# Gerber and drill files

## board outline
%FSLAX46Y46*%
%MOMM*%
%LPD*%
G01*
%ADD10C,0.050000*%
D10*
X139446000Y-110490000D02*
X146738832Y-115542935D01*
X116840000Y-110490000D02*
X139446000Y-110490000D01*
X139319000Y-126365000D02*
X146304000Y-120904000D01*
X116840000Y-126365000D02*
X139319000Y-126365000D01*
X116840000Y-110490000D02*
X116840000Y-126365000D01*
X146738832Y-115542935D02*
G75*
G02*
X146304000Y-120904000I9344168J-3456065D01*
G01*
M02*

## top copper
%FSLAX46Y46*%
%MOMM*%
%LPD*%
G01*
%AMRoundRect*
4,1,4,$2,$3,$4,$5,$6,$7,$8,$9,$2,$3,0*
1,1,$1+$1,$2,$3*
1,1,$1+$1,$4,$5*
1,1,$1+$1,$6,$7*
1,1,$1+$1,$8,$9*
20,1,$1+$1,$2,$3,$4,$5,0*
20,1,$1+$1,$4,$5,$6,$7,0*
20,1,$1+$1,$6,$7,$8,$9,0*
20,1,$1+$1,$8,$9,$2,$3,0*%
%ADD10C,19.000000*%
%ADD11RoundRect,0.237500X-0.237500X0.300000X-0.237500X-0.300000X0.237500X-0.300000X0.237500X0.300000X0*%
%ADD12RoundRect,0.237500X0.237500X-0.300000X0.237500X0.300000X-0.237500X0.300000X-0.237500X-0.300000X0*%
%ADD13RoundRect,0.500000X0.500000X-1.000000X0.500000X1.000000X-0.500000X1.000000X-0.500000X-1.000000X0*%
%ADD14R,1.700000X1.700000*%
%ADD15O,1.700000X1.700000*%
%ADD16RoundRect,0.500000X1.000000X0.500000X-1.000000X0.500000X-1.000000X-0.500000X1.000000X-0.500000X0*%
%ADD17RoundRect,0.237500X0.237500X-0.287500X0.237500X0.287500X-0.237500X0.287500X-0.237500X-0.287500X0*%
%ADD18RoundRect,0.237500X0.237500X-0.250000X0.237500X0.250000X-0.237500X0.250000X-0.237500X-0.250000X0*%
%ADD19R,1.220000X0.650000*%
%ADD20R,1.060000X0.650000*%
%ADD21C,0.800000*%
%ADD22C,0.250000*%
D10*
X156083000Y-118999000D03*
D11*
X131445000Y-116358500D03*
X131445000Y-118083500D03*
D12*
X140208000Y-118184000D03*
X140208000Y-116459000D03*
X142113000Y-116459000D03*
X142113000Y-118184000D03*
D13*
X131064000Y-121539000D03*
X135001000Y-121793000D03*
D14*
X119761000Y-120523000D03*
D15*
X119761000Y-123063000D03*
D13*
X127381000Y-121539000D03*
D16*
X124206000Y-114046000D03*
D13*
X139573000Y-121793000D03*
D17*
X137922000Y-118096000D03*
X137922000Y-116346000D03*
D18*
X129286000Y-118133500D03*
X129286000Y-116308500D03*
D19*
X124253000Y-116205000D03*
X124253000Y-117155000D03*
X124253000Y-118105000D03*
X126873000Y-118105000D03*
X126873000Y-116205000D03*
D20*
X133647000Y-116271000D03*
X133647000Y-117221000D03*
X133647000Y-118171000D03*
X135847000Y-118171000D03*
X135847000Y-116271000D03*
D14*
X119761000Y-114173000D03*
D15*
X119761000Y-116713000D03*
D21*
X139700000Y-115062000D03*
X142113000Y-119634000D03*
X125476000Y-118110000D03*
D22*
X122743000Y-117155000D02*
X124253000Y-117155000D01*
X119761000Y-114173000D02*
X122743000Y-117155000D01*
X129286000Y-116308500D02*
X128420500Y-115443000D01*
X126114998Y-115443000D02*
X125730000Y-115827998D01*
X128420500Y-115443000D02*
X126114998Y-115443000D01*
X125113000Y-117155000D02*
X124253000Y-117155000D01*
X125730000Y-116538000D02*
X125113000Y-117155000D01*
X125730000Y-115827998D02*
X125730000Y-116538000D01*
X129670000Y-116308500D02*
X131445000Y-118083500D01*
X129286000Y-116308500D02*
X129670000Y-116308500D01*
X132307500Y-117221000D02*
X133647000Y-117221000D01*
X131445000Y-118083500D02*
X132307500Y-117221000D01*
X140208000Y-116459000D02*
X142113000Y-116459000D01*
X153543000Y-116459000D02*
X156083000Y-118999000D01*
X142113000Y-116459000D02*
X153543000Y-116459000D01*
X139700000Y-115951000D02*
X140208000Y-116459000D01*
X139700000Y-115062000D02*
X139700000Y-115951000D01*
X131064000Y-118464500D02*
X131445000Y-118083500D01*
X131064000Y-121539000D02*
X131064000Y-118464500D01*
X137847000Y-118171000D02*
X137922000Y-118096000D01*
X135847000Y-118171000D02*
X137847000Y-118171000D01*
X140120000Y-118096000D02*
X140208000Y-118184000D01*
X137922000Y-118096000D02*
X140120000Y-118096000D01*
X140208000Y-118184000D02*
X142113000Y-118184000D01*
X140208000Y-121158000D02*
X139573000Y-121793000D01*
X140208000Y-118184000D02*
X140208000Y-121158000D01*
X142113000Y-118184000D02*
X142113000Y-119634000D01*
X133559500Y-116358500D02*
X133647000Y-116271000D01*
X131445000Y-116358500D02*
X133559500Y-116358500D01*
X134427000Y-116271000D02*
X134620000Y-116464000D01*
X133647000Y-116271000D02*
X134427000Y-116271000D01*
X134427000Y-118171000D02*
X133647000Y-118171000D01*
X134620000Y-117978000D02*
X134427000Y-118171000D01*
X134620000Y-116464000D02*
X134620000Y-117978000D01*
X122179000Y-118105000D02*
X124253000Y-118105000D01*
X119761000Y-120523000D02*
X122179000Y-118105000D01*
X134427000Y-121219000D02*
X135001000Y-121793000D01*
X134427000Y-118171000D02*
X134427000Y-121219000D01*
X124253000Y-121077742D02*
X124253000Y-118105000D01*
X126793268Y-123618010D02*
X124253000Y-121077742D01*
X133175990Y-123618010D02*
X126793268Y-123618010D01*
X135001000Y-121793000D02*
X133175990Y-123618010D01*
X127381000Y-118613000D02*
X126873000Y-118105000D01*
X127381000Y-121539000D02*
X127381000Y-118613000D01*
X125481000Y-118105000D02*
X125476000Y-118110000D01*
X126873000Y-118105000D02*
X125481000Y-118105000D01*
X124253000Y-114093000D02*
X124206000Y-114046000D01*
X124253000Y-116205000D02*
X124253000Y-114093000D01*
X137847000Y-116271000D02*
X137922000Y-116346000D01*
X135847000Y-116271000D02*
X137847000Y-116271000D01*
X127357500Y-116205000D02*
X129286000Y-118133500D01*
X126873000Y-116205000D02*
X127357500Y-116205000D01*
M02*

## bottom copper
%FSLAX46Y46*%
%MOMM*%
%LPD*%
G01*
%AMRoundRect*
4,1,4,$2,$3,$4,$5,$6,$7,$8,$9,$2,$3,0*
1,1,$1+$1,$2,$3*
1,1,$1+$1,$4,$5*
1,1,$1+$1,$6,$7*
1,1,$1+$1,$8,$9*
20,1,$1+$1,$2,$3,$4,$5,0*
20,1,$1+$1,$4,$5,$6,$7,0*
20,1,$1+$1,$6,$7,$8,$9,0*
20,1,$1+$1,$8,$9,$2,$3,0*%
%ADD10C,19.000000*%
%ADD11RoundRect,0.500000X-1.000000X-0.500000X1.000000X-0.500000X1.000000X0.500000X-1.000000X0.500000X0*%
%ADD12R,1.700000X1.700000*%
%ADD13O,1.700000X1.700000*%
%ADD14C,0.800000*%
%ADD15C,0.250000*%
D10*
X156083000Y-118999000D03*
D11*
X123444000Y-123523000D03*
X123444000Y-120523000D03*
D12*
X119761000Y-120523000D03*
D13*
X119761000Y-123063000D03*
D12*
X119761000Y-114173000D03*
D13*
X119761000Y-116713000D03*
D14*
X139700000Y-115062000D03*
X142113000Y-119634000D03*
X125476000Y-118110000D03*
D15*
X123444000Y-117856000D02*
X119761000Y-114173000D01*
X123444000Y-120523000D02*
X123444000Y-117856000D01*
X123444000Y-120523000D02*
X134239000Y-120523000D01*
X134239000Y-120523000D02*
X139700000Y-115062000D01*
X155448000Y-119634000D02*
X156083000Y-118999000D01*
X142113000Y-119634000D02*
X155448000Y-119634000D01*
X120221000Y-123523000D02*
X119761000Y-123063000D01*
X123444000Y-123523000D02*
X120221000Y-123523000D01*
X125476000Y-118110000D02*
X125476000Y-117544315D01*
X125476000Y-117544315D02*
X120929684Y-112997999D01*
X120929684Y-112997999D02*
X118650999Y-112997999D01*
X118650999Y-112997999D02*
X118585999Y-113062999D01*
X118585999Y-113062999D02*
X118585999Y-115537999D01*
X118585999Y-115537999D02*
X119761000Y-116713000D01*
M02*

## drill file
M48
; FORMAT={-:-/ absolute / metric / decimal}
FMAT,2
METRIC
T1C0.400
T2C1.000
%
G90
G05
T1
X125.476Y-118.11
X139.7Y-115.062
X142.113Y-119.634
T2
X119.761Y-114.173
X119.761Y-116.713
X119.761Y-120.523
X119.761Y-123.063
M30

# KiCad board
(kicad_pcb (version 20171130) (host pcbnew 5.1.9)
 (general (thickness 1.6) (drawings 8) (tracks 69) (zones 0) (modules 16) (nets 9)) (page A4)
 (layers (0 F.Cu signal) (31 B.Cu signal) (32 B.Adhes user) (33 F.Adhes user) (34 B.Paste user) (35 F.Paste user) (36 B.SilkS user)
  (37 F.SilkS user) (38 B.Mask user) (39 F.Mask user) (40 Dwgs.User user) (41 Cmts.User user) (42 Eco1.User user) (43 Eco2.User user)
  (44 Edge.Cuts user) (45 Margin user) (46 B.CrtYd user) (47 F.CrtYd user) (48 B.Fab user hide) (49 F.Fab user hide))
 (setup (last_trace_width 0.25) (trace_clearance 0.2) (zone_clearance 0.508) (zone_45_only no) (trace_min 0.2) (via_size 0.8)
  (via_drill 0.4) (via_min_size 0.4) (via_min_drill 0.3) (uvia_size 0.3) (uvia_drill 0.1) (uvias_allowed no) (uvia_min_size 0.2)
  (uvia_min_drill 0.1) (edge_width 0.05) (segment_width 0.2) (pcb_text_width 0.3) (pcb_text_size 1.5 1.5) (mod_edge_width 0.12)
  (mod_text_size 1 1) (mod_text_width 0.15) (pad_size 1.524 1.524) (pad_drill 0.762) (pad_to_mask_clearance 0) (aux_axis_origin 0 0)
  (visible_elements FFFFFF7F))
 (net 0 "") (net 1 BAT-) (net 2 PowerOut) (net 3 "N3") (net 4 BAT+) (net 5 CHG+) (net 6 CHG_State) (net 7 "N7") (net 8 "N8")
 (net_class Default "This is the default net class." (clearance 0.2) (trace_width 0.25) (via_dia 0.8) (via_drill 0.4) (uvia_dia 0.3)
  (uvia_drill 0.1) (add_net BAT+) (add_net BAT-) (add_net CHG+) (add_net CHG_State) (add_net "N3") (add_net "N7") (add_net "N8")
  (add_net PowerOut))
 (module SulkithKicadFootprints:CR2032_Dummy (layer F.Cu) (at 156.083 118.999)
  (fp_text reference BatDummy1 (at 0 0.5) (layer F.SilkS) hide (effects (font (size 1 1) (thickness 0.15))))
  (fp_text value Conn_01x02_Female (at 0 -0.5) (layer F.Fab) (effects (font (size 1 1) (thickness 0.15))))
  (pad 1 smd circle (at 0 0) (size 19 19) (layers F.Cu F.Paste F.Mask) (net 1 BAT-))
  (pad 2 smd circle (at 0 0) (size 19 19) (layers B.Cu B.Paste B.Mask) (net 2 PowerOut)))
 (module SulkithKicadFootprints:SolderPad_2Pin (layer B.Cu) (at 123.444 123.523)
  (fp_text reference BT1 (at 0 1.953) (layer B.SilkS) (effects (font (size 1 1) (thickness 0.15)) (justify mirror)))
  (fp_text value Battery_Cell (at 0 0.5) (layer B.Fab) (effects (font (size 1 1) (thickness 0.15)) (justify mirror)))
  (pad 1 smd roundrect (at 0 0) (size 3 2) (layers B.Cu B.Paste B.Mask) (roundrect_rratio 0.25) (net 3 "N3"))
  (pad 2 smd roundrect (at 0 -3) (size 3 2) (layers B.Cu B.Paste B.Mask) (roundrect_rratio 0.25) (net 1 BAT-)))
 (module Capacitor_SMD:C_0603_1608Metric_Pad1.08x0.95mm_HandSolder (layer F.Cu) (at 131.445 117.221 270)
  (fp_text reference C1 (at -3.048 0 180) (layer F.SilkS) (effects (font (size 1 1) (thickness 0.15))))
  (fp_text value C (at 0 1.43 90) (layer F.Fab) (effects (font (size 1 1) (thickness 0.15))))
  (pad 1 smd roundrect (at -0.8625 0 270) (size 1.075 0.95) (layers F.Cu F.Paste F.Mask) (roundrect_rratio 0.25) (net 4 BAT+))
  (pad 2 smd roundrect (at 0.8625 0 270) (size 1.075 0.95) (layers F.Cu F.Paste F.Mask) (roundrect_rratio 0.25) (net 1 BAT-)))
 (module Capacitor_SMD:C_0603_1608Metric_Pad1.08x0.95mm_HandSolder (layer F.Cu) (at 140.208 117.3215 90)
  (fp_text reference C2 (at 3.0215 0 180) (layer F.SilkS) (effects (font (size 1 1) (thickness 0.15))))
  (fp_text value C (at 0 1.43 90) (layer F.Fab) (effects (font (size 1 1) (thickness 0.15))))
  (pad 1 smd roundrect (at -0.8625 0 90) (size 1.075 0.95) (layers F.Cu F.Paste F.Mask) (roundrect_rratio 0.25) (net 2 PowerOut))
  (pad 2 smd roundrect (at 0.8625 0 90) (size 1.075 0.95) (layers F.Cu F.Paste F.Mask) (roundrect_rratio 0.25) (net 1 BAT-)))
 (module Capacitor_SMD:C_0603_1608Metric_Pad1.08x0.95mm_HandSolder (layer F.Cu) (at 142.113 117.3215 90)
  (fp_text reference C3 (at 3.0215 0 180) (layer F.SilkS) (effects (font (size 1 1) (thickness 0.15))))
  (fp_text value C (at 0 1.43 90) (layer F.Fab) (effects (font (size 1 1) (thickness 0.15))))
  (pad 2 smd roundrect (at 0.8625 0 90) (size 1.075 0.95) (layers F.Cu F.Paste F.Mask) (roundrect_rratio 0.25) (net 1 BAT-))
  (pad 1 smd roundrect (at -0.8625 0 90) (size 1.075 0.95) (layers F.Cu F.Paste F.Mask) (roundrect_rratio 0.25) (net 2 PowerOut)))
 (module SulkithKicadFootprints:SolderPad (layer F.Cu) (at 131.064 121.539 90)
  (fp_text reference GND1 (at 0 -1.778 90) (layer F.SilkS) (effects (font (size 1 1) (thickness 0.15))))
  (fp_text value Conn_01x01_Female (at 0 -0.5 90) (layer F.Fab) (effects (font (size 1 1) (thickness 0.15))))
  (pad 1 smd roundrect (at 0 0 90) (size 3 2) (layers F.Cu F.Paste F.Mask) (roundrect_rratio 0.25) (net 1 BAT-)))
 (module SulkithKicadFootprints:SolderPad (layer F.Cu) (at 135.001 121.793 90)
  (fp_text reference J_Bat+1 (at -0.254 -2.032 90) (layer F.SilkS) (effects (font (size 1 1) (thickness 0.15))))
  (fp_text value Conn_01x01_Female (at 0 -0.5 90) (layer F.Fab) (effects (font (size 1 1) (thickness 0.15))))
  (pad 1 smd roundrect (at 0 0 90) (size 3 2) (layers F.Cu F.Paste F.Mask) (roundrect_rratio 0.25) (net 4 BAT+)))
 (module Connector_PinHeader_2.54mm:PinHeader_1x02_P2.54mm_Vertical (layer F.Cu) (at 119.761 120.523)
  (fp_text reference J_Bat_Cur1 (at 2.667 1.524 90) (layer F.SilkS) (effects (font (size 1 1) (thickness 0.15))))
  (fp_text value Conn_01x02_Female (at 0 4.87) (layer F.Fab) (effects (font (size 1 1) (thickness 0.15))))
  (pad 1 thru_hole rect (at 0 0) (size 1.7 1.7) (drill 1) (layers *.Cu *.Mask) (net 4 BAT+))
  (pad 2 thru_hole oval (at 0 2.54) (size 1.7 1.7) (drill 1) (layers *.Cu *.Mask) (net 3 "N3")))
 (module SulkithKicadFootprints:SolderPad (layer F.Cu) (at 127.381 121.539 90)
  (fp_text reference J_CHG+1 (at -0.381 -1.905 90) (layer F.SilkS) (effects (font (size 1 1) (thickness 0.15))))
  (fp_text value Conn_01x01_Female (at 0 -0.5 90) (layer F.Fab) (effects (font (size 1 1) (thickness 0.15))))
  (pad 1 smd roundrect (at 0 0 90) (size 3 2) (layers F.Cu F.Paste F.Mask) (roundrect_rratio 0.25) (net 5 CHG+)))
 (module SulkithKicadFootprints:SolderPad (layer F.Cu) (at 124.206 114.046 180)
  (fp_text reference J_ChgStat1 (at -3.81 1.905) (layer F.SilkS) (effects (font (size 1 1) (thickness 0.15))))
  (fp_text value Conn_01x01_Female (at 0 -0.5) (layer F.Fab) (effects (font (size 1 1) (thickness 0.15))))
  (pad 1 smd roundrect (at 0 0 180) (size 3 2) (layers F.Cu F.Paste F.Mask) (roundrect_rratio 0.25) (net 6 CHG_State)))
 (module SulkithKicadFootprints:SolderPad (layer F.Cu) (at 139.573 121.793 90)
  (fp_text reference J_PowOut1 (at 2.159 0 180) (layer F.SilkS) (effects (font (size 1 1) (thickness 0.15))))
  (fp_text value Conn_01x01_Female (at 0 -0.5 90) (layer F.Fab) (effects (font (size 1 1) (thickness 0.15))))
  (pad 1 smd roundrect (at 0 0 90) (size 3 2) (layers F.Cu F.Paste F.Mask) (roundrect_rratio 0.25) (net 2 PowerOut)))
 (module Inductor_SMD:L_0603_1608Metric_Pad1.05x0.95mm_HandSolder (layer F.Cu) (at 137.922 117.221 90)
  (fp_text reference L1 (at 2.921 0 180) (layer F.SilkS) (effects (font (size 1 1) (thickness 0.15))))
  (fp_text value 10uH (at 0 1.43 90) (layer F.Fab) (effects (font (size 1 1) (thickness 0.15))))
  (pad 1 smd roundrect (at -0.875 0 90) (size 1.05 0.95) (layers F.Cu F.Paste F.Mask) (roundrect_rratio 0.25) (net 2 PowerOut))
  (pad 2 smd roundrect (at 0.875 0 90) (size 1.05 0.95) (layers F.Cu F.Paste F.Mask) (roundrect_rratio 0.25) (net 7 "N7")))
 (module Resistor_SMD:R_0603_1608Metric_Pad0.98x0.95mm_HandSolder (layer F.Cu) (at 129.286 117.221 90)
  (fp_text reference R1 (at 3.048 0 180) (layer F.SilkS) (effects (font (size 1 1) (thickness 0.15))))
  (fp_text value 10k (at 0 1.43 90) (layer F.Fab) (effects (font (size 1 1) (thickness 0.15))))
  (pad 1 smd roundrect (at -0.9125 0 90) (size 0.975 0.95) (layers F.Cu F.Paste F.Mask) (roundrect_rratio 0.25) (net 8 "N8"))
  (pad 2 smd roundrect (at 0.9125 0 90) (size 0.975 0.95) (layers F.Cu F.Paste F.Mask) (roundrect_rratio 0.25) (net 1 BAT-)))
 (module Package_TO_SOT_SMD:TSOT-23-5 (layer F.Cu) (at 125.563 117.155)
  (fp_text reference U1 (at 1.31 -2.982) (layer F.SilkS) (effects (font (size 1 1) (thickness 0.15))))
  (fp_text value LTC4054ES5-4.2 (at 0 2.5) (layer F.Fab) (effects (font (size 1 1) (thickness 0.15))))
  (pad 1 smd rect (at -1.31 -0.95) (size 1.22 0.65) (layers F.Cu F.Paste F.Mask) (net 6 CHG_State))
  (pad 2 smd rect (at -1.31 0) (size 1.22 0.65) (layers F.Cu F.Paste F.Mask) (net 1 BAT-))
  (pad 3 smd rect (at -1.31 0.95) (size 1.22 0.65) (layers F.Cu F.Paste F.Mask) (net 4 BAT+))
  (pad 4 smd rect (at 1.31 0.95) (size 1.22 0.65) (layers F.Cu F.Paste F.Mask) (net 5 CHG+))
  (pad 5 smd rect (at 1.31 -0.95) (size 1.22 0.65) (layers F.Cu F.Paste F.Mask) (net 8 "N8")))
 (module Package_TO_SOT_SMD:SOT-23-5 (layer F.Cu) (at 134.747 117.221)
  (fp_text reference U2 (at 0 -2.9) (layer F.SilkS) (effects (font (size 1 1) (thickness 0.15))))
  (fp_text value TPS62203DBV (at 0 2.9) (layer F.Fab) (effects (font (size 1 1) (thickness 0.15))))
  (pad 1 smd rect (at -1.1 -0.95) (size 1.06 0.65) (layers F.Cu F.Paste F.Mask) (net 4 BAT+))
  (pad 2 smd rect (at -1.1 0) (size 1.06 0.65) (layers F.Cu F.Paste F.Mask) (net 1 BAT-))
  (pad 3 smd rect (at -1.1 0.95) (size 1.06 0.65) (layers F.Cu F.Paste F.Mask) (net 4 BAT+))
  (pad 4 smd rect (at 1.1 0.95) (size 1.06 0.65) (layers F.Cu F.Paste F.Mask) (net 2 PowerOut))
  (pad 5 smd rect (at 1.1 -0.95) (size 1.06 0.65) (layers F.Cu F.Paste F.Mask) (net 7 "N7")))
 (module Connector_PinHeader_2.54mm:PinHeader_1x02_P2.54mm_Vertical (layer F.Cu) (at 119.761 114.173)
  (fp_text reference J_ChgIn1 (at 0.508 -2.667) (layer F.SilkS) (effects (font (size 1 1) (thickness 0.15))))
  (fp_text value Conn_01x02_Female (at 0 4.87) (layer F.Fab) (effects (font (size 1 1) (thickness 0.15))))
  (pad 1 thru_hole rect (at 0 0) (size 1.7 1.7) (drill 1) (layers *.Cu *.Mask) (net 1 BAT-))
  (pad 2 thru_hole oval (at 0 2.54) (size 1.7 1.7) (drill 1) (layers *.Cu *.Mask) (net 5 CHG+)))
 (gr_line (start 139.446 110.49) (end 146.738832 115.542935) (layer Edge.Cuts) (width 0.05))
 (gr_line (start 116.84 110.49) (end 139.446 110.49) (layer Edge.Cuts) (width 0.05))
 (gr_line (start 139.319 126.365) (end 146.304 120.904) (layer Edge.Cuts) (width 0.05))
 (gr_line (start 116.84 126.365) (end 139.319 126.365) (layer Edge.Cuts) (width 0.05))
 (gr_line (start 116.84 110.49) (end 116.84 126.365) (layer Edge.Cuts) (width 0.05))
 (gr_arc (start 156.083 118.999) (end 146.304 120.904) (angle -328.6789588) (layer Edge.Cuts) (width 0.05))
 (segment (start 122.743 117.155) (end 124.253 117.155) (width 0.25) (layer F.Cu) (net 1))
 (segment (start 119.761 114.173) (end 122.743 117.155) (width 0.25) (layer F.Cu) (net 1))
 (segment (start 129.286 116.3085) (end 128.4205 115.443) (width 0.25) (layer F.Cu) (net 1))
 (segment (start 126.114998 115.443) (end 125.73 115.827998) (width 0.25) (layer F.Cu) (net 1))
 (segment (start 128.4205 115.443) (end 126.114998 115.443) (width 0.25) (layer F.Cu) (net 1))
 (segment (start 125.113 117.155) (end 124.253 117.155) (width 0.25) (layer F.Cu) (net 1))
 (segment (start 125.73 116.538) (end 125.113 117.155) (width 0.25) (layer F.Cu) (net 1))
 (segment (start 125.73 115.827998) (end 125.73 116.538) (width 0.25) (layer F.Cu) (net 1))
 (segment (start 129.67 116.3085) (end 131.445 118.0835) (width 0.25) (layer F.Cu) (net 1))
 (segment (start 129.286 116.3085) (end 129.67 116.3085) (width 0.25) (layer F.Cu) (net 1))
 (segment (start 132.3075 117.221) (end 133.647 117.221) (width 0.25) (layer F.Cu) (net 1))
 (segment (start 131.445 118.0835) (end 132.3075 117.221) (width 0.25) (layer F.Cu) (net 1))
 (segment (start 123.444 117.856) (end 119.761 114.173) (width 0.25) (layer B.Cu) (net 1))
 (segment (start 123.444 120.523) (end 123.444 117.856) (width 0.25) (layer B.Cu) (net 1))
 (segment (start 140.208 116.459) (end 142.113 116.459) (width 0.25) (layer F.Cu) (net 1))
 (segment (start 153.543 116.459) (end 156.083 118.999) (width 0.25) (layer F.Cu) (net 1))
 (segment (start 142.113 116.459) (end 153.543 116.459) (width 0.25) (layer F.Cu) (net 1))
 (segment (start 123.444 120.523) (end 134.239 120.523) (width 0.25) (layer B.Cu) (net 1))
 (via (at 139.7 115.062) (size 0.8) (drill 0.4) (layers F.Cu B.Cu) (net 1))
 (segment (start 134.239 120.523) (end 139.7 115.062) (width 0.25) (layer B.Cu) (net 1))
 (segment (start 139.7 115.951) (end 140.208 116.459) (width 0.25) (layer F.Cu) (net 1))
 (segment (start 139.7 115.062) (end 139.7 115.951) (width 0.25) (layer F.Cu) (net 1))
 (segment (start 131.064 118.4645) (end 131.445 118.0835) (width 0.25) (layer F.Cu) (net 1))
 (segment (start 131.064 121.539) (end 131.064 118.4645) (width 0.25) (layer F.Cu) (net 1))
 (segment (start 137.847 118.171) (end 137.922 118.096) (width 0.25) (layer F.Cu) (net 2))
 (segment (start 135.847 118.171) (end 137.847 118.171) (width 0.25) (layer F.Cu) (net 2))
 (segment (start 140.12 118.096) (end 140.208 118.184) (width 0.25) (layer F.Cu) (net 2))
 (segment (start 137.922 118.096) (end 140.12 118.096) (width 0.25) (layer F.Cu) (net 2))
 (segment (start 140.208 118.184) (end 142.113 118.184) (width 0.25) (layer F.Cu) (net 2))
 (segment (start 140.208 121.158) (end 139.573 121.793) (width 0.25) (layer F.Cu) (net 2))
 (segment (start 140.208 118.184) (end 140.208 121.158) (width 0.25) (layer F.Cu) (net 2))
 (via (at 142.113 119.634) (size 0.8) (drill 0.4) (layers F.Cu B.Cu) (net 2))
 (segment (start 142.113 118.184) (end 142.113 119.634) (width 0.25) (layer F.Cu) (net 2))
 (segment (start 155.448 119.634) (end 156.083 118.999) (width 0.25) (layer B.Cu) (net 2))
 (segment (start 142.113 119.634) (end 155.448 119.634) (width 0.25) (layer B.Cu) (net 2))
 (segment (start 120.221 123.523) (end 119.761 123.063) (width 0.25) (layer B.Cu) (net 3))
 (segment (start 123.444 123.523) (end 120.221 123.523) (width 0.25) (layer B.Cu) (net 3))
 (segment (start 133.5595 116.3585) (end 133.647 116.271) (width 0.25) (layer F.Cu) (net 4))
 (segment (start 131.445 116.3585) (end 133.5595 116.3585) (width 0.25) (layer F.Cu) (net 4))
 (segment (start 134.427 116.271) (end 134.62 116.464) (width 0.25) (layer F.Cu) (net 4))
 (segment (start 133.647 116.271) (end 134.427 116.271) (width 0.25) (layer F.Cu) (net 4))
 (segment (start 134.427 118.171) (end 133.647 118.171) (width 0.25) (layer F.Cu) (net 4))
 (segment (start 134.62 117.978) (end 134.427 118.171) (width 0.25) (layer F.Cu) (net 4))
 (segment (start 134.62 116.464) (end 134.62 117.978) (width 0.25) (layer F.Cu) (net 4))
 (segment (start 122.179 118.105) (end 124.253 118.105) (width 0.25) (layer F.Cu) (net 4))
 (segment (start 119.761 120.523) (end 122.179 118.105) (width 0.25) (layer F.Cu) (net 4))
 (segment (start 134.427 121.219) (end 135.001 121.793) (width 0.25) (layer F.Cu) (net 4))
 (segment (start 134.427 118.171) (end 134.427 121.219) (width 0.25) (layer F.Cu) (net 4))
 (segment (start 124.253 121.077742) (end 124.253 118.105) (width 0.25) (layer F.Cu) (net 4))
 (segment (start 126.793268 123.61801) (end 124.253 121.077742) (width 0.25) (layer F.Cu) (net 4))
 (segment (start 133.17599 123.61801) (end 126.793268 123.61801) (width 0.25) (layer F.Cu) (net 4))
 (segment (start 135.001 121.793) (end 133.17599 123.61801) (width 0.25) (layer F.Cu) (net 4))
 (segment (start 127.381 118.613) (end 126.873 118.105) (width 0.25) (layer F.Cu) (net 5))
 (segment (start 127.381 121.539) (end 127.381 118.613) (width 0.25) (layer F.Cu) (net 5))
 (via (at 125.476 118.11) (size 0.8) (drill 0.4) (layers F.Cu B.Cu) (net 5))
 (segment (start 125.481 118.105) (end 125.476 118.11) (width 0.25) (layer F.Cu) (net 5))
 (segment (start 126.873 118.105) (end 125.481 118.105) (width 0.25) (layer F.Cu) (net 5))
 (segment (start 125.476 118.11) (end 125.476 117.544315) (width 0.25) (layer B.Cu) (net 5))
 (segment (start 125.476 117.544315) (end 120.929684 112.997999) (width 0.25) (layer B.Cu) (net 5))
 (segment (start 120.929684 112.997999) (end 118.650999 112.997999) (width 0.25) (layer B.Cu) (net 5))
 (segment (start 118.650999 112.997999) (end 118.585999 113.062999) (width 0.25) (layer B.Cu) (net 5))
 (segment (start 118.585999 113.062999) (end 118.585999 115.537999) (width 0.25) (layer B.Cu) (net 5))
 (segment (start 118.585999 115.537999) (end 119.761 116.713) (width 0.25) (layer B.Cu) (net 5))
 (segment (start 124.253 114.093) (end 124.206 114.046) (width 0.25) (layer F.Cu) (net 6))
 (segment (start 124.253 116.205) (end 124.253 114.093) (width 0.25) (layer F.Cu) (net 6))
 (segment (start 137.847 116.271) (end 137.922 116.346) (width 0.25) (layer F.Cu) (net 7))
 (segment (start 135.847 116.271) (end 137.847 116.271) (width 0.25) (layer F.Cu) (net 7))
 (segment (start 127.3575 116.205) (end 129.286 118.1335) (width 0.25) (layer F.Cu) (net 8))
 (segment (start 126.873 116.205) (end 127.3575 116.205) (width 0.25) (layer F.Cu) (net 8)))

